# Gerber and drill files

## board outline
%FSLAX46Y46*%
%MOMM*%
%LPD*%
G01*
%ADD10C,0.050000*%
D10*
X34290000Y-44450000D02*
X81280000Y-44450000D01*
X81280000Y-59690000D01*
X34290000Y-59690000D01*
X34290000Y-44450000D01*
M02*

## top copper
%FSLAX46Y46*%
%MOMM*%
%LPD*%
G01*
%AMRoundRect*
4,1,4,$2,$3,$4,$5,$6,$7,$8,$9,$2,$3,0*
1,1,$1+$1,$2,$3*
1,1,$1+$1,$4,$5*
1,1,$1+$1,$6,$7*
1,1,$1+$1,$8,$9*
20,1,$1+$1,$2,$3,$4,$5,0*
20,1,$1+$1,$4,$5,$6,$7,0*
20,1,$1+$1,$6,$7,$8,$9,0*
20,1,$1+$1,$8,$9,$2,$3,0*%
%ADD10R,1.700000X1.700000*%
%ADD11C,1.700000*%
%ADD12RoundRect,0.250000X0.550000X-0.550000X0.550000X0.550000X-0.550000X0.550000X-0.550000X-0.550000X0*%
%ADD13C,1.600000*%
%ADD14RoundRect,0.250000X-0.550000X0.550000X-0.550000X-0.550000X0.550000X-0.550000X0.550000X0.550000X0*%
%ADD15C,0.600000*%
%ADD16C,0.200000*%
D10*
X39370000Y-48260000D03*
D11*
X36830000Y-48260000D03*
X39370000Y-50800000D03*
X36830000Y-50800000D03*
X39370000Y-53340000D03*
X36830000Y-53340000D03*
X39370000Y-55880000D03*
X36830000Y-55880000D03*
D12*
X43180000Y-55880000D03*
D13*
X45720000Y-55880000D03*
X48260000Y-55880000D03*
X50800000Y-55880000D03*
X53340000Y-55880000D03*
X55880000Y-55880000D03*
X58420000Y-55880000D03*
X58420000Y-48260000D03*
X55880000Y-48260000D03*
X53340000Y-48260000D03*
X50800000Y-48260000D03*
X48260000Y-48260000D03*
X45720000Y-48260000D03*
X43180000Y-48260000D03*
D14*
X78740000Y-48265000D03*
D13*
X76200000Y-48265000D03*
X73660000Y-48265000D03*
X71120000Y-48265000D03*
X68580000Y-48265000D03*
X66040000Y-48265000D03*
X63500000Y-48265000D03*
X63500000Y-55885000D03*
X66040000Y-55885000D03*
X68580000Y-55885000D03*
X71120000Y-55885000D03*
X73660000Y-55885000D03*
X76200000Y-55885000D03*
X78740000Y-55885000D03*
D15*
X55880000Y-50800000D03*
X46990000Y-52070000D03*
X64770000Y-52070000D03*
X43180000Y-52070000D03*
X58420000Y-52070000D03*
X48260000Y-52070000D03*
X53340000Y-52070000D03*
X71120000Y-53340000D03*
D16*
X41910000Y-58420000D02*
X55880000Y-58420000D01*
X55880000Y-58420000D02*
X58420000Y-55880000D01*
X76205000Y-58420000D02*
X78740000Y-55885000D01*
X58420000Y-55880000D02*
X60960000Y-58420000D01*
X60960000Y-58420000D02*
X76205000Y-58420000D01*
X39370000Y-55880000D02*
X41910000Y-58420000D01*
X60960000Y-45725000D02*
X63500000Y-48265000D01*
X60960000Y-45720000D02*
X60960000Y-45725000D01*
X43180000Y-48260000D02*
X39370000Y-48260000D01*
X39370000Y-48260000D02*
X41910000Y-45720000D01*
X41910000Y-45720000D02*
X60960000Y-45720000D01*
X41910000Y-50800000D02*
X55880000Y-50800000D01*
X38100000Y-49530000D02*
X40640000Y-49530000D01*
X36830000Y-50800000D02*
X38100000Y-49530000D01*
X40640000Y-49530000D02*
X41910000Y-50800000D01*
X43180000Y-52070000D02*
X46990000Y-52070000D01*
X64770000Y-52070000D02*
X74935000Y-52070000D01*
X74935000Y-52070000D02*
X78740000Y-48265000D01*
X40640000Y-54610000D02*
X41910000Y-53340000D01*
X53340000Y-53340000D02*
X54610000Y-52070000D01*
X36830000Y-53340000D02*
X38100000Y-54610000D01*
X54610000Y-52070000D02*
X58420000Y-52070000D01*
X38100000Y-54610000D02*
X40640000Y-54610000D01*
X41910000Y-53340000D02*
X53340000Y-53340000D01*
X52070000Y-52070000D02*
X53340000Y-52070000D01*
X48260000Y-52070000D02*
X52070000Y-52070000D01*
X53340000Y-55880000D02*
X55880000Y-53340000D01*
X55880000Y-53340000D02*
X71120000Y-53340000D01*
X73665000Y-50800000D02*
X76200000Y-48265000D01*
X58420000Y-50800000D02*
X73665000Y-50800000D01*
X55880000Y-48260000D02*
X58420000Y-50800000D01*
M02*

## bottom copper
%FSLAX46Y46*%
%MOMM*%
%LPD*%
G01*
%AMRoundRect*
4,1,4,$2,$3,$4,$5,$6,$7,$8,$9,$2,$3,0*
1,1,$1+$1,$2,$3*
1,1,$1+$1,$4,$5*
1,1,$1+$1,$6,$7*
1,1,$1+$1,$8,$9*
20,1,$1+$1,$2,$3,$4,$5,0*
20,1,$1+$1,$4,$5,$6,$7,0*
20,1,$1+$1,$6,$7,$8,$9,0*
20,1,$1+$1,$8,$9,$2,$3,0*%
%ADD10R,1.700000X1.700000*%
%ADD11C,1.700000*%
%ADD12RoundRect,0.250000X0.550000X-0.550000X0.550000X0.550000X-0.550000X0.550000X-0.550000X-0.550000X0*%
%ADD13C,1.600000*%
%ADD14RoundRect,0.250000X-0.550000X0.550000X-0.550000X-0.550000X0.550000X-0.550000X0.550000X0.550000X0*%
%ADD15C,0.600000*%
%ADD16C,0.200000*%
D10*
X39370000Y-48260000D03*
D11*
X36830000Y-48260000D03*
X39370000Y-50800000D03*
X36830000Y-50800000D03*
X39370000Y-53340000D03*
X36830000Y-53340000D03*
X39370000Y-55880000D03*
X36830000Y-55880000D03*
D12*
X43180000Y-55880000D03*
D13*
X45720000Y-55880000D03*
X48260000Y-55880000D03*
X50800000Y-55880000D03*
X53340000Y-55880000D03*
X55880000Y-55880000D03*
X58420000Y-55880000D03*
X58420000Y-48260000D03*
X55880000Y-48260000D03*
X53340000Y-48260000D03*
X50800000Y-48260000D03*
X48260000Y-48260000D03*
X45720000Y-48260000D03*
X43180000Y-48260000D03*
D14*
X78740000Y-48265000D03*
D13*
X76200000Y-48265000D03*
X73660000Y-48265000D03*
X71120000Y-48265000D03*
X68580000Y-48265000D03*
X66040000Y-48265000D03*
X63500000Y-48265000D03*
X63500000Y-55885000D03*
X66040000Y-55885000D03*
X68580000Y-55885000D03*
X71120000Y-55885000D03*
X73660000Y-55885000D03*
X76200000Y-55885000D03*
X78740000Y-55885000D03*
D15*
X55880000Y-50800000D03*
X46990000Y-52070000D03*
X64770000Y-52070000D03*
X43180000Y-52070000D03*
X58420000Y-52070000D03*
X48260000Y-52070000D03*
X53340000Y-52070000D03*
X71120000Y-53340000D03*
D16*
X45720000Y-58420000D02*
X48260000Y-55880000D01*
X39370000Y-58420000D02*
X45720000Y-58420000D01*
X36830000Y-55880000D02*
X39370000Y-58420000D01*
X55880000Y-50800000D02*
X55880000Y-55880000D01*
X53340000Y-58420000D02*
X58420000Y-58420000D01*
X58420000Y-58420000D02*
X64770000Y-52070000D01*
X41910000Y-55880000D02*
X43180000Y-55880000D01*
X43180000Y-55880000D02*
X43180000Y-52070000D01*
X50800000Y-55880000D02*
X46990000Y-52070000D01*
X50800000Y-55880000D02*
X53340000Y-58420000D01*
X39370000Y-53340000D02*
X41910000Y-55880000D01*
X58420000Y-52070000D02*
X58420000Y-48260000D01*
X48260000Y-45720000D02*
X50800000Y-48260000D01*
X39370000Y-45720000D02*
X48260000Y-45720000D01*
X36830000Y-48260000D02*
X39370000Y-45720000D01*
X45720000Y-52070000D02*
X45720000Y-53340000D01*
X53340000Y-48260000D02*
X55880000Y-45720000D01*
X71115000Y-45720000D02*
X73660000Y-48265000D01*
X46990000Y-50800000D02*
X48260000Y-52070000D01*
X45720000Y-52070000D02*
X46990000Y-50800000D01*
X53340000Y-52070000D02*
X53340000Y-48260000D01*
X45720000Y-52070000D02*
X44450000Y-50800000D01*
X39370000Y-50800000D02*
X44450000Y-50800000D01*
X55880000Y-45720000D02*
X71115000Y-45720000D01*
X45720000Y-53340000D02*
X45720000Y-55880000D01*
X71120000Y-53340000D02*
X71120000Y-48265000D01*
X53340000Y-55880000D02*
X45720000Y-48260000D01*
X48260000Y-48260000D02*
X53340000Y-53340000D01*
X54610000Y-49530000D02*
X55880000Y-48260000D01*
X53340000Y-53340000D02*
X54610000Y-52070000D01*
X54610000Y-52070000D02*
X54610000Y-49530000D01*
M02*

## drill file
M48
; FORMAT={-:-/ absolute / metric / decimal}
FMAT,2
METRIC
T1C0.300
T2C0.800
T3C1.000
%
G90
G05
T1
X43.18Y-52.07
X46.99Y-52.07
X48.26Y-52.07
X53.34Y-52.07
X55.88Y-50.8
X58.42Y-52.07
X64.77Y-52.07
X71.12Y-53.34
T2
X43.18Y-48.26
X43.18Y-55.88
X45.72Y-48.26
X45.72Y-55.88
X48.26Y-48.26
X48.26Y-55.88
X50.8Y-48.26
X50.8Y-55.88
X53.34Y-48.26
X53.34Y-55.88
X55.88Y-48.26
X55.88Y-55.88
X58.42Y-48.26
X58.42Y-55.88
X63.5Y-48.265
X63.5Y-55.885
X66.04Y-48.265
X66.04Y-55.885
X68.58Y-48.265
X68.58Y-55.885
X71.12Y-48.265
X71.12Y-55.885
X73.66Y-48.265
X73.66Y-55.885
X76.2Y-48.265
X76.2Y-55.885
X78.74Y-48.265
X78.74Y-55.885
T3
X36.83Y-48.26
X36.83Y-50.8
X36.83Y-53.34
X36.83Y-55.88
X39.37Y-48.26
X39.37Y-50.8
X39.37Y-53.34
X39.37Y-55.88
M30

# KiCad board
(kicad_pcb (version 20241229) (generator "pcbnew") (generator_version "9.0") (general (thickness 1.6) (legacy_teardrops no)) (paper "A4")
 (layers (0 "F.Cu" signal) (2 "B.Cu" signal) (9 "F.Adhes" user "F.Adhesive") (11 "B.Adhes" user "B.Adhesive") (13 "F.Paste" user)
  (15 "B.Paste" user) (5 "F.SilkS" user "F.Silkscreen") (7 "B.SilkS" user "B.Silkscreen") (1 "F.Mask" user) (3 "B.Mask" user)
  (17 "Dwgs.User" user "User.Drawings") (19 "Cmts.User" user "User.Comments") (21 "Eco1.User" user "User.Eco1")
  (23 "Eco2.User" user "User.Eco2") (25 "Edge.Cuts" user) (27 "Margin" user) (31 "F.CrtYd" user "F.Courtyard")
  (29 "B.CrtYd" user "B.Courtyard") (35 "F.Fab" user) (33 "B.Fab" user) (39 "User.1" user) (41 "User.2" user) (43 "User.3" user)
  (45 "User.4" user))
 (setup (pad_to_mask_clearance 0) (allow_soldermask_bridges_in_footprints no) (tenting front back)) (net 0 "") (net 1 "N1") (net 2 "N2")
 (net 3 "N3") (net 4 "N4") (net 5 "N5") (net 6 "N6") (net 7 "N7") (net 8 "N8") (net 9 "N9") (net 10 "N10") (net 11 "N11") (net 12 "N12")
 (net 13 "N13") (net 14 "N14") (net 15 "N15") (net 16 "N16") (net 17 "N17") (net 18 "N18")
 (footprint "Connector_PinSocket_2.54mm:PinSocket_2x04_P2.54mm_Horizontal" (layer "F.Cu") (at 39.37 48.26)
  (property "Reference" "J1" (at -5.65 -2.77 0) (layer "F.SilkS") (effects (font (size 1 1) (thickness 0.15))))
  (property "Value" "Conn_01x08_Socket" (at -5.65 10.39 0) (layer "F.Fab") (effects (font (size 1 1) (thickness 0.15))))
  (pad "1" thru_hole rect (at 0 0) (size 1.7 1.7) (drill 1) (layers "*.Cu" "*.Mask") (remove_unused_layers no) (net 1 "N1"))
  (pad "2" thru_hole circle (at -2.54 0) (size 1.7 1.7) (drill 1) (layers "*.Cu" "*.Mask") (remove_unused_layers no) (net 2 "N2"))
  (pad "3" thru_hole circle (at 0 2.54) (size 1.7 1.7) (drill 1) (layers "*.Cu" "*.Mask") (remove_unused_layers no) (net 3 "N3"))
  (pad "4" thru_hole circle (at -2.54 2.54) (size 1.7 1.7) (drill 1) (layers "*.Cu" "*.Mask") (remove_unused_layers no) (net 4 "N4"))
  (pad "5" thru_hole circle (at 0 5.08) (size 1.7 1.7) (drill 1) (layers "*.Cu" "*.Mask") (remove_unused_layers no) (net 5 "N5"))
  (pad "6" thru_hole circle (at -2.54 5.08) (size 1.7 1.7) (drill 1) (layers "*.Cu" "*.Mask") (remove_unused_layers no) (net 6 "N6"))
  (pad "7" thru_hole circle (at 0 7.62) (size 1.7 1.7) (drill 1) (layers "*.Cu" "*.Mask") (remove_unused_layers no) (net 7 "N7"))
  (pad "8" thru_hole circle (at -2.54 7.62) (size 1.7 1.7) (drill 1) (layers "*.Cu" "*.Mask") (remove_unused_layers no) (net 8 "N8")))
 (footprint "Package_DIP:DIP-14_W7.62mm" (layer "F.Cu") (at 43.18 55.88 90)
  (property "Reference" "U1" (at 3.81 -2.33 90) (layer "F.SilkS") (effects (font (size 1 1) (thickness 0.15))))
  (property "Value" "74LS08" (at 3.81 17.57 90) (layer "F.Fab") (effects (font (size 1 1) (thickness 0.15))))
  (pad "1" thru_hole roundrect (at 0 0 90) (size 1.6 1.6) (drill 0.8) (layers "*.Cu" "*.Mask") (remove_unused_layers no)
   (roundrect_rratio 0.15625) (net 5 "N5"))
  (pad "2" thru_hole circle (at 0 2.54 90) (size 1.6 1.6) (drill 0.8) (layers "*.Cu" "*.Mask") (remove_unused_layers no) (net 3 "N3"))
  (pad "3" thru_hole circle (at 0 5.08 90) (size 1.6 1.6) (drill 0.8) (layers "*.Cu" "*.Mask") (remove_unused_layers no) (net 8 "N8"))
  (pad "4" thru_hole circle (at 0 7.62 90) (size 1.6 1.6) (drill 0.8) (layers "*.Cu" "*.Mask") (remove_unused_layers no) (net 5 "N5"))
  (pad "5" thru_hole circle (at 0 10.16 90) (size 1.6 1.6) (drill 0.8) (layers "*.Cu" "*.Mask") (remove_unused_layers no) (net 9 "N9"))
  (pad "6" thru_hole circle (at 0 12.7 90) (size 1.6 1.6) (drill 0.8) (layers "*.Cu" "*.Mask") (remove_unused_layers no) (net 4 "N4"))
  (pad "7" thru_hole circle (at 0 15.24 90) (size 1.6 1.6) (drill 0.8) (layers "*.Cu" "*.Mask") (remove_unused_layers no) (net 7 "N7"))
  (pad "8" thru_hole circle (at 7.62 15.24 90) (size 1.6 1.6) (drill 0.8) (layers "*.Cu" "*.Mask") (remove_unused_layers no) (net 6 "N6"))
  (pad "9" thru_hole circle (at 7.62 12.7 90) (size 1.6 1.6) (drill 0.8) (layers "*.Cu" "*.Mask") (remove_unused_layers no) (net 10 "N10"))
  (pad "10" thru_hole circle (at 7.62 10.16 90) (size 1.6 1.6) (drill 0.8) (layers "*.Cu" "*.Mask") (remove_unused_layers no) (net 3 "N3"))
  (pad "11" thru_hole circle (at 7.62 7.62 90) (size 1.6 1.6) (drill 0.8) (layers "*.Cu" "*.Mask") (remove_unused_layers no) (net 2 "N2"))
  (pad "12" thru_hole circle (at 7.62 5.08 90) (size 1.6 1.6) (drill 0.8) (layers "*.Cu" "*.Mask") (remove_unused_layers no) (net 10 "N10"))
  (pad "13" thru_hole circle (at 7.62 2.54 90) (size 1.6 1.6) (drill 0.8) (layers "*.Cu" "*.Mask") (remove_unused_layers no) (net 9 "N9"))
  (pad "14" thru_hole circle (at 7.62 0 90) (size 1.6 1.6) (drill 0.8) (layers "*.Cu" "*.Mask") (remove_unused_layers no) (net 1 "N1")))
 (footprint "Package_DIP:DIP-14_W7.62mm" (layer "F.Cu") (at 78.74 48.265 -90)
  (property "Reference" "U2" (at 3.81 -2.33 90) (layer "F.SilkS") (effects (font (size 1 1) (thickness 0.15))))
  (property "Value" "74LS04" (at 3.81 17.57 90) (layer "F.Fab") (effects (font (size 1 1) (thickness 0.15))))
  (pad "1" thru_hole roundrect (at 0 0 270) (size 1.6 1.6) (drill 0.8) (layers "*.Cu" "*.Mask") (remove_unused_layers no)
   (roundrect_rratio 0.15625) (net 5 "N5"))
  (pad "2" thru_hole circle (at 0 2.54 270) (size 1.6 1.6) (drill 0.8) (layers "*.Cu" "*.Mask") (remove_unused_layers no) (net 10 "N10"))
  (pad "3" thru_hole circle (at 0 5.08 270) (size 1.6 1.6) (drill 0.8) (layers "*.Cu" "*.Mask") (remove_unused_layers no) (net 3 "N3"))
  (pad "4" thru_hole circle (at 0 7.62 270) (size 1.6 1.6) (drill 0.8) (layers "*.Cu" "*.Mask") (remove_unused_layers no) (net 9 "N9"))
  (pad "5" thru_hole circle (at 0 10.16 270) (size 1.6 1.6) (drill 0.8) (layers "*.Cu" "*.Mask") (remove_unused_layers no) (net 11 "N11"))
  (pad "6" thru_hole circle (at 0 12.7 270) (size 1.6 1.6) (drill 0.8) (layers "*.Cu" "*.Mask") (remove_unused_layers no) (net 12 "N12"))
  (pad "7" thru_hole circle (at 0 15.24 270) (size 1.6 1.6) (drill 0.8) (layers "*.Cu" "*.Mask") (remove_unused_layers no) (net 1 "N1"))
  (pad "8" thru_hole circle (at 7.62 15.24 270) (size 1.6 1.6) (drill 0.8) (layers "*.Cu" "*.Mask") (remove_unused_layers no) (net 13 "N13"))
  (pad "9" thru_hole circle (at 7.62 12.7 270) (size 1.6 1.6) (drill 0.8) (layers "*.Cu" "*.Mask") (remove_unused_layers no) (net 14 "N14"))
  (pad "10" thru_hole circle (at 7.62 10.16 270) (size 1.6 1.6) (drill 0.8) (layers "*.Cu" "*.Mask") (remove_unused_layers no)
   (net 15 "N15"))
  (pad "11" thru_hole circle (at 7.62 7.62 270) (size 1.6 1.6) (drill 0.8) (layers "*.Cu" "*.Mask") (remove_unused_layers no) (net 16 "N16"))
  (pad "12" thru_hole circle (at 7.62 5.08 270) (size 1.6 1.6) (drill 0.8) (layers "*.Cu" "*.Mask") (remove_unused_layers no) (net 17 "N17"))
  (pad "13" thru_hole circle (at 7.62 2.54 270) (size 1.6 1.6) (drill 0.8) (layers "*.Cu" "*.Mask") (remove_unused_layers no) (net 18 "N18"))
  (pad "14" thru_hole circle (at 7.62 0 270) (size 1.6 1.6) (drill 0.8) (layers "*.Cu" "*.Mask") (remove_unused_layers no) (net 7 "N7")))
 (gr_rect (start 34.29 44.45) (end 81.28 59.69) (stroke (width 0.05) (type default)) (fill no) (layer "Edge.Cuts"))
 (segment (start 45.72 58.42) (end 48.26 55.88) (width 0.2) (layer "B.Cu") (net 8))
 (segment (start 39.37 58.42) (end 45.72 58.42) (width 0.2) (layer "B.Cu") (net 8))
 (segment (start 36.83 55.88) (end 39.37 58.42) (width 0.2) (layer "B.Cu") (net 8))
 (segment (start 41.91 58.42) (end 55.88 58.42) (width 0.2) (layer "F.Cu") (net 7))
 (segment (start 55.88 58.42) (end 58.42 55.88) (width 0.2) (layer "F.Cu") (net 7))
 (segment (start 76.205 58.42) (end 78.74 55.885) (width 0.2) (layer "F.Cu") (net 7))
 (segment (start 58.42 55.88) (end 60.96 58.42) (width 0.2) (layer "F.Cu") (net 7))
 (segment (start 60.96 58.42) (end 76.205 58.42) (width 0.2) (layer "F.Cu") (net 7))
 (segment (start 39.37 55.88) (end 41.91 58.42) (width 0.2) (layer "F.Cu") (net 7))
 (segment (start 60.96 45.725) (end 63.5 48.265) (width 0.2) (layer "F.Cu") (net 1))
 (segment (start 60.96 45.72) (end 60.96 45.725) (width 0.2) (layer "F.Cu") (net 1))
 (segment (start 43.18 48.26) (end 39.37 48.26) (width 0.2) (layer "F.Cu") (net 1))
 (segment (start 39.37 48.26) (end 41.91 45.72) (width 0.2) (layer "F.Cu") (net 1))
 (segment (start 41.91 45.72) (end 60.96 45.72) (width 0.2) (layer "F.Cu") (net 1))
 (segment (start 41.91 50.8) (end 55.88 50.8) (width 0.2) (layer "F.Cu") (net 4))
 (segment (start 38.1 49.53) (end 40.64 49.53) (width 0.2) (layer "F.Cu") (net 4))
 (segment (start 36.83 50.8) (end 38.1 49.53) (width 0.2) (layer "F.Cu") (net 4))
 (segment (start 40.64 49.53) (end 41.91 50.8) (width 0.2) (layer "F.Cu") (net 4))
 (via (at 55.88 50.8) (size 0.6) (drill 0.3) (layers "F.Cu" "B.Cu") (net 4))
 (segment (start 55.88 50.8) (end 55.88 55.88) (width 0.2) (layer "B.Cu") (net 4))
 (segment (start 43.18 52.07) (end 46.99 52.07) (width 0.2) (layer "F.Cu") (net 5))
 (segment (start 64.77 52.07) (end 74.935 52.07) (width 0.2) (layer "F.Cu") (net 5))
 (segment (start 74.935 52.07) (end 78.74 48.265) (width 0.2) (layer "F.Cu") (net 5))
 (via (at 46.99 52.07) (size 0.6) (drill 0.3) (layers "F.Cu" "B.Cu") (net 5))
 (via (at 64.77 52.07) (size 0.6) (drill 0.3) (layers "F.Cu" "B.Cu") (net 5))
 (via (at 43.18 52.07) (size 0.6) (drill 0.3) (layers "F.Cu" "B.Cu") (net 5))
 (segment (start 53.34 58.42) (end 58.42 58.42) (width 0.2) (layer "B.Cu") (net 5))
 (segment (start 58.42 58.42) (end 64.77 52.07) (width 0.2) (layer "B.Cu") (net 5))
 (segment (start 41.91 55.88) (end 43.18 55.88) (width 0.2) (layer "B.Cu") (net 5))
 (segment (start 43.18 55.88) (end 43.18 52.07) (width 0.2) (layer "B.Cu") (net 5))
 (segment (start 50.8 55.88) (end 46.99 52.07) (width 0.2) (layer "B.Cu") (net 5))
 (segment (start 50.8 55.88) (end 53.34 58.42) (width 0.2) (layer "B.Cu") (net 5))
 (segment (start 39.37 53.34) (end 41.91 55.88) (width 0.2) (layer "B.Cu") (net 5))
 (segment (start 40.64 54.61) (end 41.91 53.34) (width 0.2) (layer "F.Cu") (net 6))
 (segment (start 53.34 53.34) (end 54.61 52.07) (width 0.2) (layer "F.Cu") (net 6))
 (segment (start 36.83 53.34) (end 38.1 54.61) (width 0.2) (layer "F.Cu") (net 6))
 (segment (start 54.61 52.07) (end 58.42 52.07) (width 0.2) (layer "F.Cu") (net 6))
 (segment (start 38.1 54.61) (end 40.64 54.61) (width 0.2) (layer "F.Cu") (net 6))
 (segment (start 41.91 53.34) (end 53.34 53.34) (width 0.2) (layer "F.Cu") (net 6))
 (via (at 58.42 52.07) (size 0.6) (drill 0.3) (layers "F.Cu" "B.Cu") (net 6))
 (segment (start 58.42 52.07) (end 58.42 48.26) (width 0.2) (layer "B.Cu") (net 6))
 (segment (start 48.26 45.72) (end 50.8 48.26) (width 0.2) (layer "B.Cu") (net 2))
 (segment (start 39.37 45.72) (end 48.26 45.72) (width 0.2) (layer "B.Cu") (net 2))
 (segment (start 36.83 48.26) (end 39.37 45.72) (width 0.2) (layer "B.Cu") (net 2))
 (segment (start 52.07 52.07) (end 53.34 52.07) (width 0.2) (layer "F.Cu") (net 3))
 (segment (start 48.26 52.07) (end 52.07 52.07) (width 0.2) (layer "F.Cu") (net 3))
 (via (at 48.26 52.07) (size 0.6) (drill 0.3) (layers "F.Cu" "B.Cu") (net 3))
 (via (at 53.34 52.07) (size 0.6) (drill 0.3) (layers "F.Cu" "B.Cu") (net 3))
 (segment (start 45.72 52.07) (end 45.72 53.34) (width 0.2) (layer "B.Cu") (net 3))
 (segment (start 53.34 48.26) (end 55.88 45.72) (width 0.2) (layer "B.Cu") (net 3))
 (segment (start 71.115 45.72) (end 73.66 48.265) (width 0.2) (layer "B.Cu") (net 3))
 (segment (start 46.99 50.8) (end 48.26 52.07) (width 0.2) (layer "B.Cu") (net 3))
 (segment (start 45.72 52.07) (end 46.99 50.8) (width 0.2) (layer "B.Cu") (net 3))
 (segment (start 53.34 52.07) (end 53.34 48.26) (width 0.2) (layer "B.Cu") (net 3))
 (segment (start 45.72 52.07) (end 44.45 50.8) (width 0.2) (layer "B.Cu") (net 3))
 (segment (start 39.37 50.8) (end 44.45 50.8) (width 0.2) (layer "B.Cu") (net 3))
 (segment (start 55.88 45.72) (end 71.115 45.72) (width 0.2) (layer "B.Cu") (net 3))
 (segment (start 45.72 53.34) (end 45.72 55.88) (width 0.2) (layer "B.Cu") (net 3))
 (segment (start 53.34 55.88) (end 55.88 53.34) (width 0.2) (layer "F.Cu") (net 9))
 (segment (start 55.88 53.34) (end 71.12 53.34) (width 0.2) (layer "F.Cu") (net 9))
 (via (at 71.12 53.34) (size 0.6) (drill 0.3) (layers "F.Cu" "B.Cu") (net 9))
 (segment (start 71.12 53.34) (end 71.12 48.265) (width 0.2) (layer "B.Cu") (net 9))
 (segment (start 53.34 55.88) (end 45.72 48.26) (width 0.2) (layer "B.Cu") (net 9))
 (segment (start 73.665 50.8) (end 76.2 48.265) (width 0.2) (layer "F.Cu") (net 10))
 (segment (start 58.42 50.8) (end 73.665 50.8) (width 0.2) (layer "F.Cu") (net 10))
 (segment (start 55.88 48.26) (end 58.42 50.8) (width 0.2) (layer "F.Cu") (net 10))
 (segment (start 48.26 48.26) (end 53.34 53.34) (width 0.2) (layer "B.Cu") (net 10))
 (segment (start 54.61 49.53) (end 55.88 48.26) (width 0.2) (layer "B.Cu") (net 10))
 (segment (start 53.34 53.34) (end 54.61 52.07) (width 0.2) (layer "B.Cu") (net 10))
 (segment (start 54.61 52.07) (end 54.61 49.53) (width 0.2) (layer "B.Cu") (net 10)))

